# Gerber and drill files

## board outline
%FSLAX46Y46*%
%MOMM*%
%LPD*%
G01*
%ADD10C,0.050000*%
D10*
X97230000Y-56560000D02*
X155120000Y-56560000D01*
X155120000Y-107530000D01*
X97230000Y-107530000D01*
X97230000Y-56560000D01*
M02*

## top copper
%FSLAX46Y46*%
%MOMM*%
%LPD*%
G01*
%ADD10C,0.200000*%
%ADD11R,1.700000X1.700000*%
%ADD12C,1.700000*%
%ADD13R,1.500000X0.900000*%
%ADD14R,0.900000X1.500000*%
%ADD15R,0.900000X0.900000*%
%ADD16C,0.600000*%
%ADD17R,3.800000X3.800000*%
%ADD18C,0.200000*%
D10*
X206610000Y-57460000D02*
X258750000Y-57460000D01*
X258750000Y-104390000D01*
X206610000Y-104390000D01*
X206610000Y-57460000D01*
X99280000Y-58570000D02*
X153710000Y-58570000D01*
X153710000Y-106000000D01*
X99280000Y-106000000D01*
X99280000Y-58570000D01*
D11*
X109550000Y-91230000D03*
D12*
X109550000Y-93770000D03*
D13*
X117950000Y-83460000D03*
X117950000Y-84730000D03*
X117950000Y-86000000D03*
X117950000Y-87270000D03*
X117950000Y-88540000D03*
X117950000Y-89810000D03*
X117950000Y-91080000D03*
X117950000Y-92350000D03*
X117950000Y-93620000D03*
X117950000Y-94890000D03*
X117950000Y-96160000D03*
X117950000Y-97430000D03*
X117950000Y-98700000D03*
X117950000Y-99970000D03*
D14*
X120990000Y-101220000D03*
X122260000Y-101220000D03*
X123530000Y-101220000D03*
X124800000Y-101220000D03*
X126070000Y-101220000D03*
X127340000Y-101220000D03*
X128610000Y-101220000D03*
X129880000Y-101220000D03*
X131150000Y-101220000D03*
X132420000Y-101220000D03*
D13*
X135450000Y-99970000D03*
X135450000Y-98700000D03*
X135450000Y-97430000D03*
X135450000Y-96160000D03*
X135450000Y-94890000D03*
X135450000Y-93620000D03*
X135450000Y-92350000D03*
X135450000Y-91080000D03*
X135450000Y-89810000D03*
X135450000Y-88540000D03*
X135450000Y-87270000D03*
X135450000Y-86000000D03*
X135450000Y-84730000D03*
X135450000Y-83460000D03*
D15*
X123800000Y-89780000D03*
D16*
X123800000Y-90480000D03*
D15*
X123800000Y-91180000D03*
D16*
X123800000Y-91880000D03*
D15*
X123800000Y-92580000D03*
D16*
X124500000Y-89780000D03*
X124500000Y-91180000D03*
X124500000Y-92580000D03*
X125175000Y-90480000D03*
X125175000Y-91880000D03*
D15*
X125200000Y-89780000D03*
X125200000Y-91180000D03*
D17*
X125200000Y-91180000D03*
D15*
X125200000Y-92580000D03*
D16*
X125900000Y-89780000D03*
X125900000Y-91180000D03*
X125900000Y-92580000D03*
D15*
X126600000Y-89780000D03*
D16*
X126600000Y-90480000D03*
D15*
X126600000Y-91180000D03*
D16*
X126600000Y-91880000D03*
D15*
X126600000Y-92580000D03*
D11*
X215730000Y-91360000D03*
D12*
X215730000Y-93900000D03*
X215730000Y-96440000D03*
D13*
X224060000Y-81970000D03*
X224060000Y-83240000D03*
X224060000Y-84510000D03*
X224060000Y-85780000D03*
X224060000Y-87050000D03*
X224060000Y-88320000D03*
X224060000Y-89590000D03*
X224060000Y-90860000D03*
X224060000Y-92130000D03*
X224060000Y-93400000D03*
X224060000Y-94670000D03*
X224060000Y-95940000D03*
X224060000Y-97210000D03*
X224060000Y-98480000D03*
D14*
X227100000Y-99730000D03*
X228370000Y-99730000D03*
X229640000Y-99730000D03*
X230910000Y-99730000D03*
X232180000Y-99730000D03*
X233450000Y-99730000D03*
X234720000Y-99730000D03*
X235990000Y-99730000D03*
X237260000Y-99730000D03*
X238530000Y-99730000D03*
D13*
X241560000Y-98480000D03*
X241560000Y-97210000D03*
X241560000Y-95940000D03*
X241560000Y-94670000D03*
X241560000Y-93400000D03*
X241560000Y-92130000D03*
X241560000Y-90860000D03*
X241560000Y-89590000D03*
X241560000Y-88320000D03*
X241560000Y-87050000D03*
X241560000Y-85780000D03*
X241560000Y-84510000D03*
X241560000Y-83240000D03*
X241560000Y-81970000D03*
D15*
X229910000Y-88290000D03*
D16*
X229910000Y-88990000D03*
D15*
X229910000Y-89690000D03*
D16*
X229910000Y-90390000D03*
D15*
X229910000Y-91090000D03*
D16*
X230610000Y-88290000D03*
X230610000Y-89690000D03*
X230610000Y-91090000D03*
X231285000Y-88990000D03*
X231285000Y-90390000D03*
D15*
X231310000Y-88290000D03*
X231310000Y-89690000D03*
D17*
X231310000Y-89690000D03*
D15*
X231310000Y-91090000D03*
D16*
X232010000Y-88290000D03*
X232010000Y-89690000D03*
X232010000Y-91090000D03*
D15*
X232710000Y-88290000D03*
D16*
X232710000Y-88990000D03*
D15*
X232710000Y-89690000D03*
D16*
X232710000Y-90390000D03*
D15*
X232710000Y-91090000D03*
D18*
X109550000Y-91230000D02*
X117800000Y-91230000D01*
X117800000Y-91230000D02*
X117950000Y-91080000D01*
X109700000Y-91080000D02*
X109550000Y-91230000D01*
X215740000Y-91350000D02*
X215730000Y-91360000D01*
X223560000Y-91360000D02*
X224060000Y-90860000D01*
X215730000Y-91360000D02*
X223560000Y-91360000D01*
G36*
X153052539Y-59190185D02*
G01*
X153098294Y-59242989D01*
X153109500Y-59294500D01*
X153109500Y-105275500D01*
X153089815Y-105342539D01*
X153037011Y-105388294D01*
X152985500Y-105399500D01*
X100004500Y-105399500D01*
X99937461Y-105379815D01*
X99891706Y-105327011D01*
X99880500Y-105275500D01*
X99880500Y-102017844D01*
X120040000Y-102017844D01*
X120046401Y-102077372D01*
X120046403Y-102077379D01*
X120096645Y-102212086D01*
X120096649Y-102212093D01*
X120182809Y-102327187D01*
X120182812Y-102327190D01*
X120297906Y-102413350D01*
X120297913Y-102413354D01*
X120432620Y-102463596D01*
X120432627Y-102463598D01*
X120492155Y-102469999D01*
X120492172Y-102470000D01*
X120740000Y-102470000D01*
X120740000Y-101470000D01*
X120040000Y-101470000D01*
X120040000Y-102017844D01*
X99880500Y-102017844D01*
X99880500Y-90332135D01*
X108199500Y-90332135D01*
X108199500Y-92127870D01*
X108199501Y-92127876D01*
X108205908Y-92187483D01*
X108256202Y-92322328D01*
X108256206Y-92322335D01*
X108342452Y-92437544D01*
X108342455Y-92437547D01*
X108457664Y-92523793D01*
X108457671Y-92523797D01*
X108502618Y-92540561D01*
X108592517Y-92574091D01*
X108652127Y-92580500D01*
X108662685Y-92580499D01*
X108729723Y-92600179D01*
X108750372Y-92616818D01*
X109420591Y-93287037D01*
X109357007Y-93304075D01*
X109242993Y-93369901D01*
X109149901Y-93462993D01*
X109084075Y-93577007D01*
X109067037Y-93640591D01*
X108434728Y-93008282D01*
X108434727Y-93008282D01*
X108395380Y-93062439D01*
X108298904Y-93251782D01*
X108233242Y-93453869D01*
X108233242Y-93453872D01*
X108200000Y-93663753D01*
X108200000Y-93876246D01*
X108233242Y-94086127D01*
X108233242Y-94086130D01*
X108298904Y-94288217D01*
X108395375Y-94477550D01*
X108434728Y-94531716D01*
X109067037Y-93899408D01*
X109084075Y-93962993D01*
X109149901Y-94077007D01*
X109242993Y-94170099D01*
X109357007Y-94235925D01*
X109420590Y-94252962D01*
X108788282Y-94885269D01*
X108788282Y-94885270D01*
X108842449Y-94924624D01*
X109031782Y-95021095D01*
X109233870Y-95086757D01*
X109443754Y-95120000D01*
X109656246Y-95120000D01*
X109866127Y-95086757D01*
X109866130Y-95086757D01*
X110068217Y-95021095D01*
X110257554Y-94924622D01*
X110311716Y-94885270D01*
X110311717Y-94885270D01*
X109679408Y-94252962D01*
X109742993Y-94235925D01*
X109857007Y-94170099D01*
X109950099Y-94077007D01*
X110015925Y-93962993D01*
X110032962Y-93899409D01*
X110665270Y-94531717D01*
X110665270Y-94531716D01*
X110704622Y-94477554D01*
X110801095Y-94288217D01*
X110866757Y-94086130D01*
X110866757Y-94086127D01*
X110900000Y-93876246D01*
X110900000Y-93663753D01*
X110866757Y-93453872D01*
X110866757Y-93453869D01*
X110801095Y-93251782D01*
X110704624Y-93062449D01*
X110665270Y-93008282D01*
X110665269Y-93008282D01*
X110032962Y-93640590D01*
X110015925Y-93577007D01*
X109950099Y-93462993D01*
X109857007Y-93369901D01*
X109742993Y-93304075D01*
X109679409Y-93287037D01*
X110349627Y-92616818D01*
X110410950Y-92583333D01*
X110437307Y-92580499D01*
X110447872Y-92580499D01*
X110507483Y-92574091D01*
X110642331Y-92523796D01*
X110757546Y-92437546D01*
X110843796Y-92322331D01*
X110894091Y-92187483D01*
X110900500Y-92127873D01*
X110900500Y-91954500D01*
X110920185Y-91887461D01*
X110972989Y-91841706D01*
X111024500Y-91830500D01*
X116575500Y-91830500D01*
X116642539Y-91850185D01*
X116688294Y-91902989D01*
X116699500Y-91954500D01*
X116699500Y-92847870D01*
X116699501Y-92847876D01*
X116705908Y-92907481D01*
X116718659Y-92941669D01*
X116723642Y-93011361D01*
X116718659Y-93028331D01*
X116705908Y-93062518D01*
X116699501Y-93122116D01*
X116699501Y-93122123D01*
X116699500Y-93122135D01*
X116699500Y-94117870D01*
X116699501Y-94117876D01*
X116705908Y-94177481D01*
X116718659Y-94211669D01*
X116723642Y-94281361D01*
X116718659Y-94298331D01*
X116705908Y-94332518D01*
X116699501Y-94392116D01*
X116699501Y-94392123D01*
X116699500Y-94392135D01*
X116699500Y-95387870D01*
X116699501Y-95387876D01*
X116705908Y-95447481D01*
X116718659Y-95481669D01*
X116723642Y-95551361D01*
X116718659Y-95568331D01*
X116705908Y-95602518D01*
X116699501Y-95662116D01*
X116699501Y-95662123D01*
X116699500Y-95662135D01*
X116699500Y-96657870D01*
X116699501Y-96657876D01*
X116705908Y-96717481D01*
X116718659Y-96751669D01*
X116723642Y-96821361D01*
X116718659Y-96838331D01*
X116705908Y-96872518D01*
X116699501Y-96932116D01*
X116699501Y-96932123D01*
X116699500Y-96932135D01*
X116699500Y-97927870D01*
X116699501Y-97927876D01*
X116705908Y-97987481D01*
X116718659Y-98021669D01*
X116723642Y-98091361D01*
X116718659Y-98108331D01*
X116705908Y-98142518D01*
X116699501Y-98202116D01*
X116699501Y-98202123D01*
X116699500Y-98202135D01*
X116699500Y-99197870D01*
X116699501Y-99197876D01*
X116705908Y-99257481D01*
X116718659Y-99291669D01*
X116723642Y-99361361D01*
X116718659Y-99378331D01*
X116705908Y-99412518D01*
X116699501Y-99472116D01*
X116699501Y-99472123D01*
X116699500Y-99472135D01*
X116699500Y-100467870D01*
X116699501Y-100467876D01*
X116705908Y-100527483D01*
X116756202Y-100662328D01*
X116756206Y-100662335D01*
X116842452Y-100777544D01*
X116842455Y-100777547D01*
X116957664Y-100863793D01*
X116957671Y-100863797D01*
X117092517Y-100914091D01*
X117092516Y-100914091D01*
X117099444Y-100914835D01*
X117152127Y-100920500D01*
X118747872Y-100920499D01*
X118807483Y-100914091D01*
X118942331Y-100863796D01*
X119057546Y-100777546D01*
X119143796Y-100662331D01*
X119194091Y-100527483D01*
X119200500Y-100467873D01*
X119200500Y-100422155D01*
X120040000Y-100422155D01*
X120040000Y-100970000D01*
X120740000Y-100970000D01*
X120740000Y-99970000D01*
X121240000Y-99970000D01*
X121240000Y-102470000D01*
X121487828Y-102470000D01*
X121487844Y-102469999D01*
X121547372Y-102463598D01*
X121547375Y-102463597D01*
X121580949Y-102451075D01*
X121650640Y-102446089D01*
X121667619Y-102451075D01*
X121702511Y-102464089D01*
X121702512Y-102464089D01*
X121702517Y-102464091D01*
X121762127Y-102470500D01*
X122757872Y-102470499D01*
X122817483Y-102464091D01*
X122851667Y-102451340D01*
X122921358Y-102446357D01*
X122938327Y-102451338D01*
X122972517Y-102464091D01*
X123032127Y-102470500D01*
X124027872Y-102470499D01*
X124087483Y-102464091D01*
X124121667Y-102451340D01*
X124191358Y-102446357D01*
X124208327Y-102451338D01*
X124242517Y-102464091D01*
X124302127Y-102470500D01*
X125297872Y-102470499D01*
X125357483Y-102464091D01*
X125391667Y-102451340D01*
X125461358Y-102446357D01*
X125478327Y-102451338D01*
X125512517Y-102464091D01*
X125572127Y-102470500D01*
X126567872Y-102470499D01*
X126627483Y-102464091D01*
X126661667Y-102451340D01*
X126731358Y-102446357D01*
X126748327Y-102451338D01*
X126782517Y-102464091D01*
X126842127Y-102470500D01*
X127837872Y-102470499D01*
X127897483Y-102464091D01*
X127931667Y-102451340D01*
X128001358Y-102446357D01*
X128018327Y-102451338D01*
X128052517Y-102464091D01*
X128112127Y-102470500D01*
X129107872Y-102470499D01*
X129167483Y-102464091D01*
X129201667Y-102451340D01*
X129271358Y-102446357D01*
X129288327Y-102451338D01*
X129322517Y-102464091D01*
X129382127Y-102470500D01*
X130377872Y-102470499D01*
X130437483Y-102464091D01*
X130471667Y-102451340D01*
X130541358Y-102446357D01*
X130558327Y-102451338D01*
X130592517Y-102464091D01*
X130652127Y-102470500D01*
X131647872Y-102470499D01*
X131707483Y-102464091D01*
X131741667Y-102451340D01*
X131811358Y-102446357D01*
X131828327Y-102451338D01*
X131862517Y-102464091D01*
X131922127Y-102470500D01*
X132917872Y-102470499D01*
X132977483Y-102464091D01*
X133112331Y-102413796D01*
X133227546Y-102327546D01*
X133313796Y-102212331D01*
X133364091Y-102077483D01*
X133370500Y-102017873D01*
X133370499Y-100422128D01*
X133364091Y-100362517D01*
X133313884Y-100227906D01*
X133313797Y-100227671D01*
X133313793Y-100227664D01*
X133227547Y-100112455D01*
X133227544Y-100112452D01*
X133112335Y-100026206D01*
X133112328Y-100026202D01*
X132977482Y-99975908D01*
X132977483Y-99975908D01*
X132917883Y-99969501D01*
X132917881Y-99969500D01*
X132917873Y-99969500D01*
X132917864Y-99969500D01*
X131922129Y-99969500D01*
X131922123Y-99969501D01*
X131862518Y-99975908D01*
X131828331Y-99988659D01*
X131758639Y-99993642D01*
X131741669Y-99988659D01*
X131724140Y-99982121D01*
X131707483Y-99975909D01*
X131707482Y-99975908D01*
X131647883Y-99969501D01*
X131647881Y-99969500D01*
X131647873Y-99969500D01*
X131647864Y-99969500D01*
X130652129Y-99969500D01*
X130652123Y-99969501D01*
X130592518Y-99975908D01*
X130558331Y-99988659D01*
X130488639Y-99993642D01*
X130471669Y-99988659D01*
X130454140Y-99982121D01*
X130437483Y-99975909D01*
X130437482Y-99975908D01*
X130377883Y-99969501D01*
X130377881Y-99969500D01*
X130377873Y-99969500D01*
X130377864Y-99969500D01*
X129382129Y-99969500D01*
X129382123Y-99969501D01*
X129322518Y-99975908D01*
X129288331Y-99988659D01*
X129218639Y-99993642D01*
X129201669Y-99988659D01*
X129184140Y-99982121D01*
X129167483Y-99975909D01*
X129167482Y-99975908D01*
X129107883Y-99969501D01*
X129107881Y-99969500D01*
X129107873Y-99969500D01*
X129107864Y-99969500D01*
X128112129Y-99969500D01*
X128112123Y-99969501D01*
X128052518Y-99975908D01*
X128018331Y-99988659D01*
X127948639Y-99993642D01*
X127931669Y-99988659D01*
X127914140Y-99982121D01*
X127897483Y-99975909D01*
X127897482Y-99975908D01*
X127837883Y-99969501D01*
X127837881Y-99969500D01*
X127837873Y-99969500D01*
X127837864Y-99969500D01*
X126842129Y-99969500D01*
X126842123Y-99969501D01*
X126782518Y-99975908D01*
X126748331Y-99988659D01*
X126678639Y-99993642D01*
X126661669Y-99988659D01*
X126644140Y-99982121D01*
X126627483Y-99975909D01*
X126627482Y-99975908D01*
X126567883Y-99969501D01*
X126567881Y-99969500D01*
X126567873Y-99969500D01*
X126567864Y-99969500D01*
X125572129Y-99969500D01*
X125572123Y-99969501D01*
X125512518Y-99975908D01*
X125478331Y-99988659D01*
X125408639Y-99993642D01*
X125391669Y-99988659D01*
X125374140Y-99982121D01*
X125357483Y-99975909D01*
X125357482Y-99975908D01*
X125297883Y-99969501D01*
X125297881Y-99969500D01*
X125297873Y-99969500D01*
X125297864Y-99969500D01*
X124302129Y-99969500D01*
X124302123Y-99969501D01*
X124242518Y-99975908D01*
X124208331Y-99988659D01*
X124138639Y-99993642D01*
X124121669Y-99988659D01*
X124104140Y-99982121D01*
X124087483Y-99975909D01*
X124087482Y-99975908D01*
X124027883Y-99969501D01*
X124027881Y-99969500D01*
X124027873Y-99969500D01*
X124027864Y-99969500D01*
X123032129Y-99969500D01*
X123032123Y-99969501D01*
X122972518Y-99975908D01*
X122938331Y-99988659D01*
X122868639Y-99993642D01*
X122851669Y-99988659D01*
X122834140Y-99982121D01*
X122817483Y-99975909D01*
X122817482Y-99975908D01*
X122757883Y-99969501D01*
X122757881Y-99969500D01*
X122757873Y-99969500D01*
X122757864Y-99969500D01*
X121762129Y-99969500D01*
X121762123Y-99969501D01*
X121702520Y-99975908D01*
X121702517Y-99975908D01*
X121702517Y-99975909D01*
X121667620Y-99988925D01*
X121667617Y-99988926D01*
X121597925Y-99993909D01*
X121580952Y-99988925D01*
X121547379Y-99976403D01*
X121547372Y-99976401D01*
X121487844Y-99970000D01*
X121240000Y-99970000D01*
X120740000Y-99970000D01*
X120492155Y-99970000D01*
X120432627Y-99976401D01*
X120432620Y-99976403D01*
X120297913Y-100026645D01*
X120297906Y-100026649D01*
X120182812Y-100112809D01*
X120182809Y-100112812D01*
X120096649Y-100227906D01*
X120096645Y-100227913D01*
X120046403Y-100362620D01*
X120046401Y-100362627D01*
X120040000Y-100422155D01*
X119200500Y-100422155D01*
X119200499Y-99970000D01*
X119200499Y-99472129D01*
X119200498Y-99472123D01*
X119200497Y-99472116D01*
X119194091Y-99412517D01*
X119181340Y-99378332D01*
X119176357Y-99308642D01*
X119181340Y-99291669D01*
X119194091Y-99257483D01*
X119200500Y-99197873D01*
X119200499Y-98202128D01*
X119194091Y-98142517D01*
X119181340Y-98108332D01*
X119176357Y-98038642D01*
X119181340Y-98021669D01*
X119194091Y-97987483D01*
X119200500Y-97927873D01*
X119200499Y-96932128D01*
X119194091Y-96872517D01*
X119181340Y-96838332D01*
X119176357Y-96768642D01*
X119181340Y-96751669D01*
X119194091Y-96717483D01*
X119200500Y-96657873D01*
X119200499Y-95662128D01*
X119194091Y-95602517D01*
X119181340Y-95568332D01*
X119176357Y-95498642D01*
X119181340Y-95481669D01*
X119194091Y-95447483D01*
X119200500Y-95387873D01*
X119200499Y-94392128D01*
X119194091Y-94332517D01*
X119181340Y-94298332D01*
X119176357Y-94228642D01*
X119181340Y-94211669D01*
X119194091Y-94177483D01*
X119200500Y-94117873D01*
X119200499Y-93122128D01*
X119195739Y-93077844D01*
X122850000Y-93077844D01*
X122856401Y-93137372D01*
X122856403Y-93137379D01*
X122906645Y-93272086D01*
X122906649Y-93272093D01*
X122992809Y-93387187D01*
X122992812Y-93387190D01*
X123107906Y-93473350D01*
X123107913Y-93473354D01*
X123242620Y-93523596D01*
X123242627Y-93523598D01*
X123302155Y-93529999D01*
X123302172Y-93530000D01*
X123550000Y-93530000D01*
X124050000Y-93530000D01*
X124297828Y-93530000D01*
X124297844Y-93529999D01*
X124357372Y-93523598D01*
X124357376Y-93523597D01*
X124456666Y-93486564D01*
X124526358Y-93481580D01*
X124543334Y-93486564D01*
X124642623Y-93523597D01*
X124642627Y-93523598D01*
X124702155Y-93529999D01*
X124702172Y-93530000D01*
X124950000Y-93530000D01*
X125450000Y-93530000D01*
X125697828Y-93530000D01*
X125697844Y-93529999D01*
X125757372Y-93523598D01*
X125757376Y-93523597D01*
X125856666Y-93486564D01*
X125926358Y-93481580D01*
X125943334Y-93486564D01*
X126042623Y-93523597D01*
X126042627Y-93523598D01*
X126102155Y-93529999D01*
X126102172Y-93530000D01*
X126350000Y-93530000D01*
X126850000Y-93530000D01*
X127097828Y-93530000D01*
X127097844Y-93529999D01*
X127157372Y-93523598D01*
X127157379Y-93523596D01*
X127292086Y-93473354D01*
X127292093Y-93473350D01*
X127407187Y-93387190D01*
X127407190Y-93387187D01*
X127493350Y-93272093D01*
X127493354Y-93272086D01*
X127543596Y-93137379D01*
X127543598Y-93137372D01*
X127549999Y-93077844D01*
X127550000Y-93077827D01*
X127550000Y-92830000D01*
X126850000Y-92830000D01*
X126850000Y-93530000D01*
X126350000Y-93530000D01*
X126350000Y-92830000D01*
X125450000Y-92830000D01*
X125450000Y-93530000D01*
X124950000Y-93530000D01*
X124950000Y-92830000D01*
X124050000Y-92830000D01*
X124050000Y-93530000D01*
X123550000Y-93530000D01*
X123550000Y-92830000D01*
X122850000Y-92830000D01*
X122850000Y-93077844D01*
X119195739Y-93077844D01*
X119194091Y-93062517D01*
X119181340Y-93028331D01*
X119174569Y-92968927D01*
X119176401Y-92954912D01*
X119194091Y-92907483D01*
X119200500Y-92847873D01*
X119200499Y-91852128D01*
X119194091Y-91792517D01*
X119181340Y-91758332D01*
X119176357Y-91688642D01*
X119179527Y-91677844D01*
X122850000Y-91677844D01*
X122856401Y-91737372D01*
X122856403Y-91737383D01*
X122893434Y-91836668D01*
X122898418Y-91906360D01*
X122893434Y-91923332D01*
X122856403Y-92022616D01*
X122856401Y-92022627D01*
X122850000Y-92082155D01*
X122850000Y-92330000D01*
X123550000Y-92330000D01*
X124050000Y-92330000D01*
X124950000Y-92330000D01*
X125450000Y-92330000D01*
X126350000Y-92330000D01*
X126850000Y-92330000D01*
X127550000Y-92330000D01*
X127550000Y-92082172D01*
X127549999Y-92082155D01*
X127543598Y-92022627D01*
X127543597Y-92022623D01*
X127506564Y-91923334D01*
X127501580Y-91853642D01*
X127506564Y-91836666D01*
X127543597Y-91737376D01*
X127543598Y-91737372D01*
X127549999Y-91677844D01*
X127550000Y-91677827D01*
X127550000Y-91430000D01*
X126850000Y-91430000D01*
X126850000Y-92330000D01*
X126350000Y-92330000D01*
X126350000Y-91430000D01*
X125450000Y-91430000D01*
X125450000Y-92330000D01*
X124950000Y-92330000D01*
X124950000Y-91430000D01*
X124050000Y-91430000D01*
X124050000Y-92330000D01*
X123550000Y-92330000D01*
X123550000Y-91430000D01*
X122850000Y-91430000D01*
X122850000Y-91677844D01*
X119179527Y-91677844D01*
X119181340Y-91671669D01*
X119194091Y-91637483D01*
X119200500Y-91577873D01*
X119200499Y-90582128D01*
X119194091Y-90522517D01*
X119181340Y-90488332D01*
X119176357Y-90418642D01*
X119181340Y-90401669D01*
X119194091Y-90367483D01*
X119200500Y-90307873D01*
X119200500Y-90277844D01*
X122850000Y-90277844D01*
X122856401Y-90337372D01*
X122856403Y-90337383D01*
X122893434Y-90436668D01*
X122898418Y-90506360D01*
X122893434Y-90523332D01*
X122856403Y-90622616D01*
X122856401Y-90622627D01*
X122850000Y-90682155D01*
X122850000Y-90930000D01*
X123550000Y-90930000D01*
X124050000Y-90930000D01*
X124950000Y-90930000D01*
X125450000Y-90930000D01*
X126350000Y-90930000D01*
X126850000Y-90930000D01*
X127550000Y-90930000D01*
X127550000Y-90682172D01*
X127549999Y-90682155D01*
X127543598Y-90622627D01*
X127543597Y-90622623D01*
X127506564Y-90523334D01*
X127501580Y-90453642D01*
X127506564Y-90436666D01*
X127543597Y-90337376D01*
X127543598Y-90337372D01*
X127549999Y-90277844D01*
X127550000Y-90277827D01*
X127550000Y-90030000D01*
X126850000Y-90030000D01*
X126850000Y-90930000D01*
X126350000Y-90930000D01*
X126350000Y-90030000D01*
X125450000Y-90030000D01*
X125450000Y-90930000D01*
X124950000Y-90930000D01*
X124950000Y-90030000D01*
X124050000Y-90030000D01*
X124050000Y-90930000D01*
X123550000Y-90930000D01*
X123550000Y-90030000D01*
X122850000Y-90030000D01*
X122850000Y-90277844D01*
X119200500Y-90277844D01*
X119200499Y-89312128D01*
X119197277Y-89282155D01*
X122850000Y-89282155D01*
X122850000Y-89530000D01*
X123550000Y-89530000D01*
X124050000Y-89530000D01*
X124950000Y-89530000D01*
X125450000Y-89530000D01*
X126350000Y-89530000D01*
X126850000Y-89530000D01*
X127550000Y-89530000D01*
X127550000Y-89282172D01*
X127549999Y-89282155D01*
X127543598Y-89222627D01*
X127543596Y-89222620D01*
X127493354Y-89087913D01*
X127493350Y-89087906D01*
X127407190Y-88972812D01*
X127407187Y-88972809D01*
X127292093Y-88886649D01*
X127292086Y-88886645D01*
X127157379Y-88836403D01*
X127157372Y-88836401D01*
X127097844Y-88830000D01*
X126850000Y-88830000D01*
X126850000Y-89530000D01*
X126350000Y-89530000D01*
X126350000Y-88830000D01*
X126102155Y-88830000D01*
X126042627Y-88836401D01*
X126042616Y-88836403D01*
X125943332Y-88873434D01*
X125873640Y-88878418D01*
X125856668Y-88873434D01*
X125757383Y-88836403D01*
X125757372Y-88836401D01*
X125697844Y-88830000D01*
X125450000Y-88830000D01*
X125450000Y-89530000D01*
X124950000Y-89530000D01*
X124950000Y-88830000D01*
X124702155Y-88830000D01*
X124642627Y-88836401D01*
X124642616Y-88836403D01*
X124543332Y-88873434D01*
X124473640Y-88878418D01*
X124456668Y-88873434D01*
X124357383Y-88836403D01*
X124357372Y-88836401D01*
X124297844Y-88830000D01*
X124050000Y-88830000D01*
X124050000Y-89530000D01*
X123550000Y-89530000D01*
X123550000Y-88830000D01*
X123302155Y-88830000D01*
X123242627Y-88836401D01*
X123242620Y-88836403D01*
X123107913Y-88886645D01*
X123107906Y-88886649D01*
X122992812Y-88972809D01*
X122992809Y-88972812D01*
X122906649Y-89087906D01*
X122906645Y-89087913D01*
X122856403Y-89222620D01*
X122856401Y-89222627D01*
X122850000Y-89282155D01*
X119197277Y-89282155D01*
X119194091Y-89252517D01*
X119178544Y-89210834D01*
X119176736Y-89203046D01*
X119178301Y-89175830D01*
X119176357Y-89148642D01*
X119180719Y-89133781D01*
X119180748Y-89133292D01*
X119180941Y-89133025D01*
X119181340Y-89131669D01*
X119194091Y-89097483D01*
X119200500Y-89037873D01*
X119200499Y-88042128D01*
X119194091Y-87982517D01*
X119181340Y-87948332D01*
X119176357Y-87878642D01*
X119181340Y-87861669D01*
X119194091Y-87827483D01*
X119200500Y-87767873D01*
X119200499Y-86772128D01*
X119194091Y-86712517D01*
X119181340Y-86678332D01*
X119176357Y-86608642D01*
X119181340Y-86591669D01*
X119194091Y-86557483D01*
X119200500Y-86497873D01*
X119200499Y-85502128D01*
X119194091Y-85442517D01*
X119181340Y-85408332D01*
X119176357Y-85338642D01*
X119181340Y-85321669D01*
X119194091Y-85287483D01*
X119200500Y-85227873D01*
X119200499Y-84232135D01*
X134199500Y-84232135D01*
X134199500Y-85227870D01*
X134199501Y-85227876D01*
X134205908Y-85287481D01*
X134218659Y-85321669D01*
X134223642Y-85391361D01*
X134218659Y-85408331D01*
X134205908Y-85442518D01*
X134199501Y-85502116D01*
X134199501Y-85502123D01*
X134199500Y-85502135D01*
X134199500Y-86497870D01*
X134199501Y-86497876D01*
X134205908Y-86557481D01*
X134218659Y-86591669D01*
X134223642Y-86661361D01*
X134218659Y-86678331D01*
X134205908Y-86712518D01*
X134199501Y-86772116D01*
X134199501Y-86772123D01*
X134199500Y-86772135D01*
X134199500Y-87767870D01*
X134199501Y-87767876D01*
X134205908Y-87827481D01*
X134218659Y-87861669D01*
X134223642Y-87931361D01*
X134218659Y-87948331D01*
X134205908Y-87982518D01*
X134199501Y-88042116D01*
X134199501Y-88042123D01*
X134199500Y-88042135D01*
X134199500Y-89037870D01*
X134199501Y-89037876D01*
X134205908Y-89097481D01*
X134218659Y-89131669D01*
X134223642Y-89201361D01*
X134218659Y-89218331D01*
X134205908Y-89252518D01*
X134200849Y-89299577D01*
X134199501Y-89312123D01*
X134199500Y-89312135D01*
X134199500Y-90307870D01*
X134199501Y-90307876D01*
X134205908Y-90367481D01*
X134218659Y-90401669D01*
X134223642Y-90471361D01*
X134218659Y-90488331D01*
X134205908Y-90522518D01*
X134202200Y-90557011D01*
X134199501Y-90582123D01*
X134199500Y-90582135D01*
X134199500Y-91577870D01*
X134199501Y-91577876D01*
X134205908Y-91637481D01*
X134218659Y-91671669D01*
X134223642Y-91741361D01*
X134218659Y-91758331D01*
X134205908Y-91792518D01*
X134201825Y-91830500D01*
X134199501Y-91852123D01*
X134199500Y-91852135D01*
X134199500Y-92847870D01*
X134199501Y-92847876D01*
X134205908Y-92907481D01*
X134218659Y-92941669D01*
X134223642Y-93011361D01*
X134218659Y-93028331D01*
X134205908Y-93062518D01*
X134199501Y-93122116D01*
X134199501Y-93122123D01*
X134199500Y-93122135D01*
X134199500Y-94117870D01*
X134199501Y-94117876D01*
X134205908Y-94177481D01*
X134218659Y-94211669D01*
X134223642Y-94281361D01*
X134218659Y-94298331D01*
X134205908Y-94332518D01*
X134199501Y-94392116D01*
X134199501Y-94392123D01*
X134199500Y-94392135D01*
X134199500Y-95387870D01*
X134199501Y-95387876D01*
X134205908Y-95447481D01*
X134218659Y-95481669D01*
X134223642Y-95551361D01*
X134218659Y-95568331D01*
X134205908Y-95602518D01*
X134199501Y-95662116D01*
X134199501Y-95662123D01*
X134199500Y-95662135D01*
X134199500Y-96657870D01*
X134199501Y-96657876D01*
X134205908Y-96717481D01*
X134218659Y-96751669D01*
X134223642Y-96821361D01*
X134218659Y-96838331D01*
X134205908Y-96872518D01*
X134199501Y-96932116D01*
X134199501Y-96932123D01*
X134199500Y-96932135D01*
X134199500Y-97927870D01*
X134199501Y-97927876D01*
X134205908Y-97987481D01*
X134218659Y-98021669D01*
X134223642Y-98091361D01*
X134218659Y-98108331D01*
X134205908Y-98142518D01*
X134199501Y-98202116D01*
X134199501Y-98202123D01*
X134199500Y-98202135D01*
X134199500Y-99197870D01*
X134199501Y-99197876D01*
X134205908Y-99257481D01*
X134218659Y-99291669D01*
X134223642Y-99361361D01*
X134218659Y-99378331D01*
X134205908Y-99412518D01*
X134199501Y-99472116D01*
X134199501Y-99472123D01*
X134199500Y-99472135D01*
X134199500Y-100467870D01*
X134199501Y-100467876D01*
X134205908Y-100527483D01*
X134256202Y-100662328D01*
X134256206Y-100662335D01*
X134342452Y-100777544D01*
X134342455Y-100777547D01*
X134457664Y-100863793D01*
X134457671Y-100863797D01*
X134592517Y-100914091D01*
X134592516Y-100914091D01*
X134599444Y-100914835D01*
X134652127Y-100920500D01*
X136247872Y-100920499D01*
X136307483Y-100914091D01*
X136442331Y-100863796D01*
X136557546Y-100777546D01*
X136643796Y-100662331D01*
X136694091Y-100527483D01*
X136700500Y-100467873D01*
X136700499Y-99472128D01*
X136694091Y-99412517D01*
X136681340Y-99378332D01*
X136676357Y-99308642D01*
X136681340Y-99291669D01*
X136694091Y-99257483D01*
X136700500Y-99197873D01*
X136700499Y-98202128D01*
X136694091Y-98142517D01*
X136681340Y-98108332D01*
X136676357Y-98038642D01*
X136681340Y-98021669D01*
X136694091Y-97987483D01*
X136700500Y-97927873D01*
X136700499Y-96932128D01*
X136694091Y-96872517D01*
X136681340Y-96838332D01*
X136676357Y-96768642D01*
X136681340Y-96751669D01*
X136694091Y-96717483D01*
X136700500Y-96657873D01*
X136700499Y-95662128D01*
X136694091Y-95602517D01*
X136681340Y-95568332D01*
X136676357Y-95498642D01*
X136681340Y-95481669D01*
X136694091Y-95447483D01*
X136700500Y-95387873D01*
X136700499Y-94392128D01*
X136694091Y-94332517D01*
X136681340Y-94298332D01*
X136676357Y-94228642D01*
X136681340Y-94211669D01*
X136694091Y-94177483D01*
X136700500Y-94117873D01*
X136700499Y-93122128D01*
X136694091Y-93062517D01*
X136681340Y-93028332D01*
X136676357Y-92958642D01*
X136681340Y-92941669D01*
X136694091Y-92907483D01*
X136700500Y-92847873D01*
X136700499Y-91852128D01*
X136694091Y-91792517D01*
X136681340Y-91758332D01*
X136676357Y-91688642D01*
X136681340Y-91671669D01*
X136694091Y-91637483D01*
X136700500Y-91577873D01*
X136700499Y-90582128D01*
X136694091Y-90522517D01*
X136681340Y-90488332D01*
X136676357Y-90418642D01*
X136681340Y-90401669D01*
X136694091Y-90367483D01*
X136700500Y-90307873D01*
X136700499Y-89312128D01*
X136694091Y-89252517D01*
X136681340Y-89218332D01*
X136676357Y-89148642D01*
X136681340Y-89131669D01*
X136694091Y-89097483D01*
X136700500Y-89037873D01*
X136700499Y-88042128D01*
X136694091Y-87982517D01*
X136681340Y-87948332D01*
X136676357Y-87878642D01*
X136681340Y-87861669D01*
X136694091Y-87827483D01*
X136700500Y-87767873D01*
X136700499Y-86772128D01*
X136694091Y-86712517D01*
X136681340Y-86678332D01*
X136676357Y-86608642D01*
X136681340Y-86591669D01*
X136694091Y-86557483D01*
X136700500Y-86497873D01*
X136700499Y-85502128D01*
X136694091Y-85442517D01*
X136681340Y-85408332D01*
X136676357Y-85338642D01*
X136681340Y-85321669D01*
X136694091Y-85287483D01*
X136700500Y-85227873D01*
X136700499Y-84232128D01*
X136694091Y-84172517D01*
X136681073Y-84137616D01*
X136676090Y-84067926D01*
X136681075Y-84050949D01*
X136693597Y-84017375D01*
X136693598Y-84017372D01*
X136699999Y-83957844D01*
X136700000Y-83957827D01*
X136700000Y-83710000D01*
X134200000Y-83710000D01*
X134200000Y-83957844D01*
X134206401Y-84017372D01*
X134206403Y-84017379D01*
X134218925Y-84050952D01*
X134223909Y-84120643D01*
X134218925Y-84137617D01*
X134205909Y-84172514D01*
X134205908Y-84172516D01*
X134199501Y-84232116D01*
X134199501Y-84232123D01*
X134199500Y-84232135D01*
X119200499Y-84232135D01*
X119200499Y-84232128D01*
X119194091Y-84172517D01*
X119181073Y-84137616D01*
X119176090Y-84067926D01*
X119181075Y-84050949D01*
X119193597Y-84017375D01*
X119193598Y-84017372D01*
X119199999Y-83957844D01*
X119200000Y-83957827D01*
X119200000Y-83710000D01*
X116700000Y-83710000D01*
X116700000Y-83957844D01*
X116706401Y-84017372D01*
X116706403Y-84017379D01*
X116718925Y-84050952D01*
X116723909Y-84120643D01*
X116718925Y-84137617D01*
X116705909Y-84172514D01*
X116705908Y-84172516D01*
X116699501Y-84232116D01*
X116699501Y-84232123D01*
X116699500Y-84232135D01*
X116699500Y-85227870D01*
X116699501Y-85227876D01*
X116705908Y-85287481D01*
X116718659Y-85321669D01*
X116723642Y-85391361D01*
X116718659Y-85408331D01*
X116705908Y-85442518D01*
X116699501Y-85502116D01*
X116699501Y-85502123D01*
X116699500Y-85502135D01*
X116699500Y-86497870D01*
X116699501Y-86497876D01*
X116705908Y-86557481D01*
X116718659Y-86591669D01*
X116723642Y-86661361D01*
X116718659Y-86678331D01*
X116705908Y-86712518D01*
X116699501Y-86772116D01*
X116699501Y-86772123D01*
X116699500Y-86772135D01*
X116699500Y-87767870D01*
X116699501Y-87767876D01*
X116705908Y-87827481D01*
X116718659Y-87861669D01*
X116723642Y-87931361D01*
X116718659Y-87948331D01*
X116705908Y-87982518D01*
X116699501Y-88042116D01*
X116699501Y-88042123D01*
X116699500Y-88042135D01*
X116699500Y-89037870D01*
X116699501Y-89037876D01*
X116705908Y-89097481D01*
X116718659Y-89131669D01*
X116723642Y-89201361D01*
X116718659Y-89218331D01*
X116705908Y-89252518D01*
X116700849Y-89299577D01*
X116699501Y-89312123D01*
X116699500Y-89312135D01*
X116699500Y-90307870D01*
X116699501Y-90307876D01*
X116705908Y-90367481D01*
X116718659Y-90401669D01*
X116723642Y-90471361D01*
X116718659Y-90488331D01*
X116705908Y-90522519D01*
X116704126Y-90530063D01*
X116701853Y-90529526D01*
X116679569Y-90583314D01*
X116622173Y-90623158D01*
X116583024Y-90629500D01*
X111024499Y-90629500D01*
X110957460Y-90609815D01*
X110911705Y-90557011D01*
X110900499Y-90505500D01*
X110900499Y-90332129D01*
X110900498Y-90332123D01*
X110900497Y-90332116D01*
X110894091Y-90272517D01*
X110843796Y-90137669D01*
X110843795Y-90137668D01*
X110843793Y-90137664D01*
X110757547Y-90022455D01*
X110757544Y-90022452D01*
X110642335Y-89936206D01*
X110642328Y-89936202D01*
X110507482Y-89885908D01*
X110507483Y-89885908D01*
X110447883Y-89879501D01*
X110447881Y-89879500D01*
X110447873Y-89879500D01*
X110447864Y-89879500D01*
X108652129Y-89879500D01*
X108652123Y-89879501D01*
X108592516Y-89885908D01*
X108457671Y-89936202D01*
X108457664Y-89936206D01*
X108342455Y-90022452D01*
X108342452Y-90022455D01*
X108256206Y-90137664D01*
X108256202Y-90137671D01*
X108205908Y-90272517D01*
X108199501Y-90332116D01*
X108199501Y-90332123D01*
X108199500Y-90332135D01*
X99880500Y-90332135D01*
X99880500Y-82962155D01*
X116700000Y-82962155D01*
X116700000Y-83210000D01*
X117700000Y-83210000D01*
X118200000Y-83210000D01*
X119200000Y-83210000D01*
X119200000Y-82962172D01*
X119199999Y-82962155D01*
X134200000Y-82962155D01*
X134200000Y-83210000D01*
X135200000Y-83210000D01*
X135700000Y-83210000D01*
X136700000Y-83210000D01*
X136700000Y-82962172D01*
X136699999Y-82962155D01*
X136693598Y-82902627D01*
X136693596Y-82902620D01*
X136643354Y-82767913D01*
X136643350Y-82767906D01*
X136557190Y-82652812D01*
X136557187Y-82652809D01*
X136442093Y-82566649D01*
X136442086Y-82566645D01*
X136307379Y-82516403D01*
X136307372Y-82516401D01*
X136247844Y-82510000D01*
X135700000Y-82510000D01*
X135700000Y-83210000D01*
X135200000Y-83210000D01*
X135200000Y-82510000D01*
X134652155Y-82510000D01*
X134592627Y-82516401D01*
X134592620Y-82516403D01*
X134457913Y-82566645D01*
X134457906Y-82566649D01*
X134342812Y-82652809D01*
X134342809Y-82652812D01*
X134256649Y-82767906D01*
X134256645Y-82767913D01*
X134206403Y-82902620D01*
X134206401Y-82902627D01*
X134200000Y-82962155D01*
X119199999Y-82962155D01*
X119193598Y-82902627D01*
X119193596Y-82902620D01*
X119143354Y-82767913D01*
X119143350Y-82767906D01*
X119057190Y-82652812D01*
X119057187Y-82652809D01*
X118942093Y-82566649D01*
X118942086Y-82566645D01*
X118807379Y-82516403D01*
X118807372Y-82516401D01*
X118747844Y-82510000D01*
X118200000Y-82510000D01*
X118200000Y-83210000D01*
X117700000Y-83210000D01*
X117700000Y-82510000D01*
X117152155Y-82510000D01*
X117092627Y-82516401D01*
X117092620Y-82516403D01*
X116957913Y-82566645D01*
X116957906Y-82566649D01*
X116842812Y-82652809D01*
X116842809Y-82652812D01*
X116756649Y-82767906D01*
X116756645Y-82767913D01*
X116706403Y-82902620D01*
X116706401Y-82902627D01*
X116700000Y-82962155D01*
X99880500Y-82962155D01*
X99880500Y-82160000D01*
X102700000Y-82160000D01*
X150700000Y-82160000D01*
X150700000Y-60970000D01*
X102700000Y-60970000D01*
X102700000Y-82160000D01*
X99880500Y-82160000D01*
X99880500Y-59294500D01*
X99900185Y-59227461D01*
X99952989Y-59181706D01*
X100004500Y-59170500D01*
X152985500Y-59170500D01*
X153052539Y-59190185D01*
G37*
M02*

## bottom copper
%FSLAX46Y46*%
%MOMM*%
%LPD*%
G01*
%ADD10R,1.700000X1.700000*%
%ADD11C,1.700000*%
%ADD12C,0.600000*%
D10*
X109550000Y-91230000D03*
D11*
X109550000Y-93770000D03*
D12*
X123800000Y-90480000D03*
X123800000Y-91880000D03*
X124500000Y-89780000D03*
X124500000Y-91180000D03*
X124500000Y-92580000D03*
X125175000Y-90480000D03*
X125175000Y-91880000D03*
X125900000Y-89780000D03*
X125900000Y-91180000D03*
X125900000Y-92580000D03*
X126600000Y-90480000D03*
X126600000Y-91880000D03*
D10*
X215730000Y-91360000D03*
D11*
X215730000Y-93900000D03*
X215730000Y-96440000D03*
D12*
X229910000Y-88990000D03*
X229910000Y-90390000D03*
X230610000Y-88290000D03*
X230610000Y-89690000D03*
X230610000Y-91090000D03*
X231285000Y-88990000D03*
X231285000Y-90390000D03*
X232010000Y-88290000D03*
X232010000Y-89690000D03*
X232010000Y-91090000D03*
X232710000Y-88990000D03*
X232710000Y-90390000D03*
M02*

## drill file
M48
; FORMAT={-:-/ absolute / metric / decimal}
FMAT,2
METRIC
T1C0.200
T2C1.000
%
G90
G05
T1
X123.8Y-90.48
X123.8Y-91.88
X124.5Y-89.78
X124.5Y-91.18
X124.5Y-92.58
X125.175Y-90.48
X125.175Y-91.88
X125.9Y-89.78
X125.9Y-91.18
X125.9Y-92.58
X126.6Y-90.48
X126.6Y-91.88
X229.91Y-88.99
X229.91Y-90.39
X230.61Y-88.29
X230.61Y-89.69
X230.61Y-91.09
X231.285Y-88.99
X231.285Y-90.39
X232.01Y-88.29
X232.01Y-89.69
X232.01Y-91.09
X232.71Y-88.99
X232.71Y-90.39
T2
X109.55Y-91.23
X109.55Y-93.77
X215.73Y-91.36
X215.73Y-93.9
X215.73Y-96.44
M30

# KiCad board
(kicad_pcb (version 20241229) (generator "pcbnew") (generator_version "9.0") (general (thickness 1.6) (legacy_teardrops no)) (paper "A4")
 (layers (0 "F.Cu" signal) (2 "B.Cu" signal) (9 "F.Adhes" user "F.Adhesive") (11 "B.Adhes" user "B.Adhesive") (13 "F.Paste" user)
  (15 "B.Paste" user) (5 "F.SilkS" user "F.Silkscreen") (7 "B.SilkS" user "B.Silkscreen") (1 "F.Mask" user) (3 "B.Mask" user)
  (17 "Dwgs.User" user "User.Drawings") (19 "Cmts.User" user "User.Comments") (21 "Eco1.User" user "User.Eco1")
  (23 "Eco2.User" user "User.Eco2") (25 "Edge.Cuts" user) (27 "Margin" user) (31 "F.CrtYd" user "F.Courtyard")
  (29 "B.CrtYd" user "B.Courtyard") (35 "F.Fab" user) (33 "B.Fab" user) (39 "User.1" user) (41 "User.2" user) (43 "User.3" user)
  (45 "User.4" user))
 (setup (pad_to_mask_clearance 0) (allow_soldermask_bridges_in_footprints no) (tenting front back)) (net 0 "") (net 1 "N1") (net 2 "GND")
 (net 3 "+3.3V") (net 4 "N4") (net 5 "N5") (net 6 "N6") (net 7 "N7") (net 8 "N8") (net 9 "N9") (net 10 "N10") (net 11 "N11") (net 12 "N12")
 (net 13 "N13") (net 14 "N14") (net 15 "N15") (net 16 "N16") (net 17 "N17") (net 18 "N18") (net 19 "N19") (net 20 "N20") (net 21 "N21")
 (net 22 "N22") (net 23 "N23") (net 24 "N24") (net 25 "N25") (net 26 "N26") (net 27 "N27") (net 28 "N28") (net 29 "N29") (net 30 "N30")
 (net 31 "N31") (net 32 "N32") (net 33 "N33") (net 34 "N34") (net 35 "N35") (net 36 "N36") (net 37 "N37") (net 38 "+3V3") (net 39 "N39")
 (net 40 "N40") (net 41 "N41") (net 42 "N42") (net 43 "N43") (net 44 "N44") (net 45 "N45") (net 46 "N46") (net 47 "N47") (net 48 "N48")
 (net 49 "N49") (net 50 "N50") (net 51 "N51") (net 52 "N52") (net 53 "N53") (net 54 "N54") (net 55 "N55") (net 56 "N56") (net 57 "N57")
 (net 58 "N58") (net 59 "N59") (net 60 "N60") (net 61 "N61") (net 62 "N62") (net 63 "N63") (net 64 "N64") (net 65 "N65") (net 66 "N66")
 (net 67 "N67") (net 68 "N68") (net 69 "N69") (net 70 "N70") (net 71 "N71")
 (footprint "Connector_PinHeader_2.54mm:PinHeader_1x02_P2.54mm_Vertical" (layer "F.Cu") (at 109.55 91.23)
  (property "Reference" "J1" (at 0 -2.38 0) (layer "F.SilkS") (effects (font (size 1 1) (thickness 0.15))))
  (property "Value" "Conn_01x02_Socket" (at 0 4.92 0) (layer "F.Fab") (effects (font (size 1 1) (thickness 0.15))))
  (pad "1" thru_hole rect (at 0 0) (size 1.7 1.7) (drill 1) (layers "*.Cu" "*.Mask") (remove_unused_layers no) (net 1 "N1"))
  (pad "2" thru_hole circle (at 0 2.54) (size 1.7 1.7) (drill 1) (layers "*.Cu" "*.Mask") (remove_unused_layers no) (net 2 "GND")))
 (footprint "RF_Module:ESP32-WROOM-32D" (layer "F.Cu") (at 126.7 91.71)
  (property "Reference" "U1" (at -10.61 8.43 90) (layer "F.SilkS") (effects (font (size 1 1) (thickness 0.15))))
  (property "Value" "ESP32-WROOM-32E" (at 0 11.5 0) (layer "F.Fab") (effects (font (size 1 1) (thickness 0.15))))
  (pad "1" smd rect (at -8.75 -8.25) (size 1.5 0.9) (layers "F.Cu" "F.Mask" "F.Paste") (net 2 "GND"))
  (pad "2" smd rect (at -8.75 -6.98) (size 1.5 0.9) (layers "F.Cu" "F.Mask" "F.Paste") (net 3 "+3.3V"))
  (pad "3" smd rect (at -8.75 -5.71) (size 1.5 0.9) (layers "F.Cu" "F.Mask" "F.Paste") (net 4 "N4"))
  (pad "4" smd rect (at -8.75 -4.44) (size 1.5 0.9) (layers "F.Cu" "F.Mask" "F.Paste") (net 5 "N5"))
  (pad "5" smd rect (at -8.75 -3.17) (size 1.5 0.9) (layers "F.Cu" "F.Mask" "F.Paste") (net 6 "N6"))
  (pad "6" smd rect (at -8.75 -1.9) (size 1.5 0.9) (layers "F.Cu" "F.Mask" "F.Paste") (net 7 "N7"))
  (pad "7" smd rect (at -8.75 -0.63) (size 1.5 0.9) (layers "F.Cu" "F.Mask" "F.Paste") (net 1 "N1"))
  (pad "8" smd rect (at -8.75 0.64) (size 1.5 0.9) (layers "F.Cu" "F.Mask" "F.Paste") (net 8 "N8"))
  (pad "9" smd rect (at -8.75 1.91) (size 1.5 0.9) (layers "F.Cu" "F.Mask" "F.Paste") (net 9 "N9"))
  (pad "10" smd rect (at -8.75 3.18) (size 1.5 0.9) (layers "F.Cu" "F.Mask" "F.Paste") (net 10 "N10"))
  (pad "11" smd rect (at -8.75 4.45) (size 1.5 0.9) (layers "F.Cu" "F.Mask" "F.Paste") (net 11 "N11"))
  (pad "12" smd rect (at -8.75 5.72) (size 1.5 0.9) (layers "F.Cu" "F.Mask" "F.Paste") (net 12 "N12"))
  (pad "13" smd rect (at -8.75 6.99) (size 1.5 0.9) (layers "F.Cu" "F.Mask" "F.Paste") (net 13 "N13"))
  (pad "14" smd rect (at -8.75 8.26) (size 1.5 0.9) (layers "F.Cu" "F.Mask" "F.Paste") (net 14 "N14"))
  (pad "15" smd rect (at -5.71 9.51 90) (size 1.5 0.9) (layers "F.Cu" "F.Mask" "F.Paste") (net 2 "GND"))
  (pad "16" smd rect (at -4.44 9.51 90) (size 1.5 0.9) (layers "F.Cu" "F.Mask" "F.Paste") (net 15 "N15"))
  (pad "17" smd rect (at -3.17 9.51 90) (size 1.5 0.9) (layers "F.Cu" "F.Mask" "F.Paste") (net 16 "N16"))
  (pad "18" smd rect (at -1.9 9.51 90) (size 1.5 0.9) (layers "F.Cu" "F.Mask" "F.Paste") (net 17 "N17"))
  (pad "19" smd rect (at -0.63 9.51 90) (size 1.5 0.9) (layers "F.Cu" "F.Mask" "F.Paste") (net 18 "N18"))
  (pad "20" smd rect (at 0.64 9.51 90) (size 1.5 0.9) (layers "F.Cu" "F.Mask" "F.Paste") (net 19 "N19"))
  (pad "21" smd rect (at 1.91 9.51 90) (size 1.5 0.9) (layers "F.Cu" "F.Mask" "F.Paste") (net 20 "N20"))
  (pad "22" smd rect (at 3.18 9.51 90) (size 1.5 0.9) (layers "F.Cu" "F.Mask" "F.Paste") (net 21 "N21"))
  (pad "23" smd rect (at 4.45 9.51 90) (size 1.5 0.9) (layers "F.Cu" "F.Mask" "F.Paste") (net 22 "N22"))
  (pad "24" smd rect (at 5.72 9.51 90) (size 1.5 0.9) (layers "F.Cu" "F.Mask" "F.Paste") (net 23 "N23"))
  (pad "25" smd rect (at 8.75 8.26) (size 1.5 0.9) (layers "F.Cu" "F.Mask" "F.Paste") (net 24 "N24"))
  (pad "26" smd rect (at 8.75 6.99) (size 1.5 0.9) (layers "F.Cu" "F.Mask" "F.Paste") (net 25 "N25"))
  (pad "27" smd rect (at 8.75 5.72) (size 1.5 0.9) (layers "F.Cu" "F.Mask" "F.Paste") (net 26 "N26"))
  (pad "28" smd rect (at 8.75 4.45) (size 1.5 0.9) (layers "F.Cu" "F.Mask" "F.Paste") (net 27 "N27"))
  (pad "29" smd rect (at 8.75 3.18) (size 1.5 0.9) (layers "F.Cu" "F.Mask" "F.Paste") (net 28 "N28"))
  (pad "30" smd rect (at 8.75 1.91) (size 1.5 0.9) (layers "F.Cu" "F.Mask" "F.Paste") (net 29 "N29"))
  (pad "31" smd rect (at 8.75 0.64) (size 1.5 0.9) (layers "F.Cu" "F.Mask" "F.Paste") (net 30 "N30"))
  (pad "32" smd rect (at 8.75 -0.63) (size 1.5 0.9) (layers "F.Cu" "F.Mask" "F.Paste") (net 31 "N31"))
  (pad "33" smd rect (at 8.75 -1.9) (size 1.5 0.9) (layers "F.Cu" "F.Mask" "F.Paste") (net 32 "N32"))
  (pad "34" smd rect (at 8.75 -3.17) (size 1.5 0.9) (layers "F.Cu" "F.Mask" "F.Paste") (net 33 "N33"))
  (pad "35" smd rect (at 8.75 -4.44) (size 1.5 0.9) (layers "F.Cu" "F.Mask" "F.Paste") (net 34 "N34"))
  (pad "36" smd rect (at 8.75 -5.71) (size 1.5 0.9) (layers "F.Cu" "F.Mask" "F.Paste") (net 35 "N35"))
  (pad "37" smd rect (at 8.75 -6.98) (size 1.5 0.9) (layers "F.Cu" "F.Mask" "F.Paste") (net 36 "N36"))
  (pad "38" smd rect (at 8.75 -8.25) (size 1.5 0.9) (layers "F.Cu" "F.Mask" "F.Paste") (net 2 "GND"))
  (pad "39" smd rect (at -2.9 -1.93) (size 0.9 0.9) (layers "F.Cu" "F.Paste") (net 2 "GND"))
  (pad "39" thru_hole circle (at -2.9 -1.23) (size 0.6 0.6) (drill 0.2) (layers "*.Cu" "F.Mask") (remove_unused_layers no) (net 2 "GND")
   (zone_connect 2))
  (pad "39" smd rect (at -2.9 -0.53) (size 0.9 0.9) (layers "F.Cu" "F.Paste") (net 2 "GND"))
  (pad "39" thru_hole circle (at -2.9 0.17) (size 0.6 0.6) (drill 0.2) (layers "*.Cu" "F.Mask") (remove_unused_layers no) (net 2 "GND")
   (zone_connect 2))
  (pad "39" smd rect (at -2.9 0.87) (size 0.9 0.9) (layers "F.Cu" "F.Paste") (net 2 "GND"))
  (pad "39" thru_hole circle (at -2.2 -1.93) (size 0.6 0.6) (drill 0.2) (layers "*.Cu" "F.Mask") (remove_unused_layers no) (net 2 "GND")
   (zone_connect 2))
  (pad "39" thru_hole circle (at -2.2 -0.53) (size 0.6 0.6) (drill 0.2) (layers "*.Cu" "F.Mask") (remove_unused_layers no) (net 2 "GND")
   (zone_connect 2))
  (pad "39" thru_hole circle (at -2.2 0.87) (size 0.6 0.6) (drill 0.2) (layers "*.Cu" "F.Mask") (remove_unused_layers no) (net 2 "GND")
   (zone_connect 2))
  (pad "39" thru_hole circle (at -1.525 -1.23) (size 0.6 0.6) (drill 0.2) (layers "*.Cu" "F.Mask") (remove_unused_layers no) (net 2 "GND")
   (zone_connect 2))
  (pad "39" thru_hole circle (at -1.525 0.17) (size 0.6 0.6) (drill 0.2) (layers "*.Cu" "F.Mask") (remove_unused_layers no) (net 2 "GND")
   (zone_connect 2))
  (pad "39" smd rect (at -1.5 -1.93) (size 0.9 0.9) (layers "F.Cu" "F.Paste") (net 2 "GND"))
  (pad "39" smd rect (at -1.5 -0.53) (size 0.9 0.9) (layers "F.Cu" "F.Paste") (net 2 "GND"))
  (pad "39" smd rect (at -1.5 -0.53) (size 3.8 3.8) (layers "F.Cu" "F.Mask") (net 2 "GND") (zone_connect 2))
  (pad "39" smd rect (at -1.5 0.87) (size 0.9 0.9) (layers "F.Cu" "F.Paste") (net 2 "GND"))
  (pad "39" thru_hole circle (at -0.8 -1.93) (size 0.6 0.6) (drill 0.2) (layers "*.Cu" "F.Mask") (remove_unused_layers no) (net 2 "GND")
   (zone_connect 2))
  (pad "39" thru_hole circle (at -0.8 -0.53) (size 0.6 0.6) (drill 0.2) (layers "*.Cu" "F.Mask") (remove_unused_layers no) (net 2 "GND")
   (zone_connect 2))
  (pad "39" thru_hole circle (at -0.8 0.87) (size 0.6 0.6) (drill 0.2) (layers "*.Cu" "F.Mask") (remove_unused_layers no) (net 2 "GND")
   (zone_connect 2))
  (pad "39" smd rect (at -0.1 -1.93) (size 0.9 0.9) (layers "F.Cu" "F.Paste") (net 2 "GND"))
  (pad "39" thru_hole circle (at -0.1 -1.23) (size 0.6 0.6) (drill 0.2) (layers "*.Cu" "F.Mask") (remove_unused_layers no) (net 2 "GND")
   (zone_connect 2))
  (pad "39" smd rect (at -0.1 -0.53) (size 0.9 0.9) (layers "F.Cu" "F.Paste") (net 2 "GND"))
  (pad "39" thru_hole circle (at -0.1 0.17) (size 0.6 0.6) (drill 0.2) (layers "*.Cu" "F.Mask") (remove_unused_layers no) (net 2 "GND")
   (zone_connect 2))
  (pad "39" smd rect (at -0.1 0.87) (size 0.9 0.9) (layers "F.Cu" "F.Paste") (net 2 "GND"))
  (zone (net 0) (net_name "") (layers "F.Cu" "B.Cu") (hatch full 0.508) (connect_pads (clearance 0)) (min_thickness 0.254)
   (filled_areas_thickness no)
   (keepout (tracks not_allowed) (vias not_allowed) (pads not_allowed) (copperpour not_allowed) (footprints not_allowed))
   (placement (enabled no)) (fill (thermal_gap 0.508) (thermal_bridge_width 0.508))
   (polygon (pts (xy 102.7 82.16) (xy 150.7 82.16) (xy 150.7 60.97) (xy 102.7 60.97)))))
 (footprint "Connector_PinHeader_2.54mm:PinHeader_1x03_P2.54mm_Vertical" (layer "F.Cu") (at 215.73 91.36)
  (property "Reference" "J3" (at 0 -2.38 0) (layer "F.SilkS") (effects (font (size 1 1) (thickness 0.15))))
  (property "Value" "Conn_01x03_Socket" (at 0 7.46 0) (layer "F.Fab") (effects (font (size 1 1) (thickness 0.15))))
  (pad "1" thru_hole rect (at 0 0) (size 1.7 1.7) (drill 1) (layers "*.Cu" "*.Mask") (remove_unused_layers no) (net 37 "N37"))
  (pad "2" thru_hole circle (at 0 2.54) (size 1.7 1.7) (drill 1) (layers "*.Cu" "*.Mask") (remove_unused_layers no) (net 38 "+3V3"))
  (pad "3" thru_hole circle (at 0 5.08) (size 1.7 1.7) (drill 1) (layers "*.Cu" "*.Mask") (remove_unused_layers no) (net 2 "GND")))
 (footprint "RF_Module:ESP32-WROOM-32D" (layer "F.Cu") (at 232.81 90.22)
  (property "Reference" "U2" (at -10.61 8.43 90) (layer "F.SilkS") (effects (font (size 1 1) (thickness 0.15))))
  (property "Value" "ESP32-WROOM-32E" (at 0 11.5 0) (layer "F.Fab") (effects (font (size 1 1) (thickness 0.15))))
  (pad "1" smd rect (at -8.75 -8.25) (size 1.5 0.9) (layers "F.Cu" "F.Mask" "F.Paste") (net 2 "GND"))
  (pad "2" smd rect (at -8.75 -6.98) (size 1.5 0.9) (layers "F.Cu" "F.Mask" "F.Paste") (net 3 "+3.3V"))
  (pad "3" smd rect (at -8.75 -5.71) (size 1.5 0.9) (layers "F.Cu" "F.Mask" "F.Paste") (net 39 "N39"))
  (pad "4" smd rect (at -8.75 -4.44) (size 1.5 0.9) (layers "F.Cu" "F.Mask" "F.Paste") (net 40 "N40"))
  (pad "5" smd rect (at -8.75 -3.17) (size 1.5 0.9) (layers "F.Cu" "F.Mask" "F.Paste") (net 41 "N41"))
  (pad "6" smd rect (at -8.75 -1.9) (size 1.5 0.9) (layers "F.Cu" "F.Mask" "F.Paste") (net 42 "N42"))
  (pad "7" smd rect (at -8.75 -0.63) (size 1.5 0.9) (layers "F.Cu" "F.Mask" "F.Paste") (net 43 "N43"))
  (pad "8" smd rect (at -8.75 0.64) (size 1.5 0.9) (layers "F.Cu" "F.Mask" "F.Paste") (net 37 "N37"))
  (pad "9" smd rect (at -8.75 1.91) (size 1.5 0.9) (layers "F.Cu" "F.Mask" "F.Paste") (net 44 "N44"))
  (pad "10" smd rect (at -8.75 3.18) (size 1.5 0.9) (layers "F.Cu" "F.Mask" "F.Paste") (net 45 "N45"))
  (pad "11" smd rect (at -8.75 4.45) (size 1.5 0.9) (layers "F.Cu" "F.Mask" "F.Paste") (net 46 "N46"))
  (pad "12" smd rect (at -8.75 5.72) (size 1.5 0.9) (layers "F.Cu" "F.Mask" "F.Paste") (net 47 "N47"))
  (pad "13" smd rect (at -8.75 6.99) (size 1.5 0.9) (layers "F.Cu" "F.Mask" "F.Paste") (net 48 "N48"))
  (pad "14" smd rect (at -8.75 8.26) (size 1.5 0.9) (layers "F.Cu" "F.Mask" "F.Paste") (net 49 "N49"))
  (pad "15" smd rect (at -5.71 9.51 90) (size 1.5 0.9) (layers "F.Cu" "F.Mask" "F.Paste") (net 2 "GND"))
  (pad "16" smd rect (at -4.44 9.51 90) (size 1.5 0.9) (layers "F.Cu" "F.Mask" "F.Paste") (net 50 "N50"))
  (pad "17" smd rect (at -3.17 9.51 90) (size 1.5 0.9) (layers "F.Cu" "F.Mask" "F.Paste") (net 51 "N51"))
  (pad "18" smd rect (at -1.9 9.51 90) (size 1.5 0.9) (layers "F.Cu" "F.Mask" "F.Paste") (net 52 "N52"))
  (pad "19" smd rect (at -0.63 9.51 90) (size 1.5 0.9) (layers "F.Cu" "F.Mask" "F.Paste") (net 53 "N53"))
  (pad "20" smd rect (at 0.64 9.51 90) (size 1.5 0.9) (layers "F.Cu" "F.Mask" "F.Paste") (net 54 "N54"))
  (pad "21" smd rect (at 1.91 9.51 90) (size 1.5 0.9) (layers "F.Cu" "F.Mask" "F.Paste") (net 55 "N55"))
  (pad "22" smd rect (at 3.18 9.51 90) (size 1.5 0.9) (layers "F.Cu" "F.Mask" "F.Paste") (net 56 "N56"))
  (pad "23" smd rect (at 4.45 9.51 90) (size 1.5 0.9) (layers "F.Cu" "F.Mask" "F.Paste") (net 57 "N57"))
  (pad "24" smd rect (at 5.72 9.51 90) (size 1.5 0.9) (layers "F.Cu" "F.Mask" "F.Paste") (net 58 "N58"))
  (pad "25" smd rect (at 8.75 8.26) (size 1.5 0.9) (layers "F.Cu" "F.Mask" "F.Paste") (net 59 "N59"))
  (pad "26" smd rect (at 8.75 6.99) (size 1.5 0.9) (layers "F.Cu" "F.Mask" "F.Paste") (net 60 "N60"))
  (pad "27" smd rect (at 8.75 5.72) (size 1.5 0.9) (layers "F.Cu" "F.Mask" "F.Paste") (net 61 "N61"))
  (pad "28" smd rect (at 8.75 4.45) (size 1.5 0.9) (layers "F.Cu" "F.Mask" "F.Paste") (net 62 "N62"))
  (pad "29" smd rect (at 8.75 3.18) (size 1.5 0.9) (layers "F.Cu" "F.Mask" "F.Paste") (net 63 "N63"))
  (pad "30" smd rect (at 8.75 1.91) (size 1.5 0.9) (layers "F.Cu" "F.Mask" "F.Paste") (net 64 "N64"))
  (pad "31" smd rect (at 8.75 0.64) (size 1.5 0.9) (layers "F.Cu" "F.Mask" "F.Paste") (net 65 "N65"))
  (pad "32" smd rect (at 8.75 -0.63) (size 1.5 0.9) (layers "F.Cu" "F.Mask" "F.Paste") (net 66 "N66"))
  (pad "33" smd rect (at 8.75 -1.9) (size 1.5 0.9) (layers "F.Cu" "F.Mask" "F.Paste") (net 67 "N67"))
  (pad "34" smd rect (at 8.75 -3.17) (size 1.5 0.9) (layers "F.Cu" "F.Mask" "F.Paste") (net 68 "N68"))
  (pad "35" smd rect (at 8.75 -4.44) (size 1.5 0.9) (layers "F.Cu" "F.Mask" "F.Paste") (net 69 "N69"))
  (pad "36" smd rect (at 8.75 -5.71) (size 1.5 0.9) (layers "F.Cu" "F.Mask" "F.Paste") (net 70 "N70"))
  (pad "37" smd rect (at 8.75 -6.98) (size 1.5 0.9) (layers "F.Cu" "F.Mask" "F.Paste") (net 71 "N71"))
  (pad "38" smd rect (at 8.75 -8.25) (size 1.5 0.9) (layers "F.Cu" "F.Mask" "F.Paste") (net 2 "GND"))
  (pad "39" smd rect (at -2.9 -1.93) (size 0.9 0.9) (layers "F.Cu" "F.Paste") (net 2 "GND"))
  (pad "39" thru_hole circle (at -2.9 -1.23) (size 0.6 0.6) (drill 0.2) (layers "*.Cu" "F.Mask") (remove_unused_layers no) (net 2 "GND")
   (zone_connect 2))
  (pad "39" smd rect (at -2.9 -0.53) (size 0.9 0.9) (layers "F.Cu" "F.Paste") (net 2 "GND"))
  (pad "39" thru_hole circle (at -2.9 0.17) (size 0.6 0.6) (drill 0.2) (layers "*.Cu" "F.Mask") (remove_unused_layers no) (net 2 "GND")
   (zone_connect 2))
  (pad "39" smd rect (at -2.9 0.87) (size 0.9 0.9) (layers "F.Cu" "F.Paste") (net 2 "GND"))
  (pad "39" thru_hole circle (at -2.2 -1.93) (size 0.6 0.6) (drill 0.2) (layers "*.Cu" "F.Mask") (remove_unused_layers no) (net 2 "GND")
   (zone_connect 2))
  (pad "39" thru_hole circle (at -2.2 -0.53) (size 0.6 0.6) (drill 0.2) (layers "*.Cu" "F.Mask") (remove_unused_layers no) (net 2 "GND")
   (zone_connect 2))
  (pad "39" thru_hole circle (at -2.2 0.87) (size 0.6 0.6) (drill 0.2) (layers "*.Cu" "F.Mask") (remove_unused_layers no) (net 2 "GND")
   (zone_connect 2))
  (pad "39" thru_hole circle (at -1.525 -1.23) (size 0.6 0.6) (drill 0.2) (layers "*.Cu" "F.Mask") (remove_unused_layers no) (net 2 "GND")
   (zone_connect 2))
  (pad "39" thru_hole circle (at -1.525 0.17) (size 0.6 0.6) (drill 0.2) (layers "*.Cu" "F.Mask") (remove_unused_layers no) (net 2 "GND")
   (zone_connect 2))
  (pad "39" smd rect (at -1.5 -1.93) (size 0.9 0.9) (layers "F.Cu" "F.Paste") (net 2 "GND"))
  (pad "39" smd rect (at -1.5 -0.53) (size 0.9 0.9) (layers "F.Cu" "F.Paste") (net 2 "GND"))
  (pad "39" smd rect (at -1.5 -0.53) (size 3.8 3.8) (layers "F.Cu" "F.Mask") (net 2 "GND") (zone_connect 2))
  (pad "39" smd rect (at -1.5 0.87) (size 0.9 0.9) (layers "F.Cu" "F.Paste") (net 2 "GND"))
  (pad "39" thru_hole circle (at -0.8 -1.93) (size 0.6 0.6) (drill 0.2) (layers "*.Cu" "F.Mask") (remove_unused_layers no) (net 2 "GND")
   (zone_connect 2))
  (pad "39" thru_hole circle (at -0.8 -0.53) (size 0.6 0.6) (drill 0.2) (layers "*.Cu" "F.Mask") (remove_unused_layers no) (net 2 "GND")
   (zone_connect 2))
  (pad "39" thru_hole circle (at -0.8 0.87) (size 0.6 0.6) (drill 0.2) (layers "*.Cu" "F.Mask") (remove_unused_layers no) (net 2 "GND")
   (zone_connect 2))
  (pad "39" smd rect (at -0.1 -1.93) (size 0.9 0.9) (layers "F.Cu" "F.Paste") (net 2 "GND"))
  (pad "39" thru_hole circle (at -0.1 -1.23) (size 0.6 0.6) (drill 0.2) (layers "*.Cu" "F.Mask") (remove_unused_layers no) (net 2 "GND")
   (zone_connect 2))
  (pad "39" smd rect (at -0.1 -0.53) (size 0.9 0.9) (layers "F.Cu" "F.Paste") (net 2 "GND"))
  (pad "39" thru_hole circle (at -0.1 0.17) (size 0.6 0.6) (drill 0.2) (layers "*.Cu" "F.Mask") (remove_unused_layers no) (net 2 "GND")
   (zone_connect 2))
  (pad "39" smd rect (at -0.1 0.87) (size 0.9 0.9) (layers "F.Cu" "F.Paste") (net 2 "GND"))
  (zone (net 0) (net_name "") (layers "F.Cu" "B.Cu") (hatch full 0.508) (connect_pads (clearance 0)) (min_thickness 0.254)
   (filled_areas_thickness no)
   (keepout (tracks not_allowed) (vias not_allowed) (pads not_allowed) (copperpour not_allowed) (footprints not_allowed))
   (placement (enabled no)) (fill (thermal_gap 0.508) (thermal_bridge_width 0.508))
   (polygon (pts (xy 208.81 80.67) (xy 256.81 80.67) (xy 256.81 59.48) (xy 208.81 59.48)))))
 (gr_rect (start 206.61 57.46) (end 258.75 104.39) (stroke (width 0.2) (type default)) (fill no) (layer "F.Cu"))
 (gr_rect (start 99.28 58.57) (end 153.71 106) (stroke (width 0.2) (type default)) (fill no) (layer "F.Cu"))
 (gr_rect (start 97.23 56.56) (end 155.12 107.53) (stroke (width 0.05) (type default)) (fill no) (layer "Edge.Cuts"))
 (segment (start 109.55 91.23) (end 117.8 91.23) (width 0.2) (layer "F.Cu") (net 1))
 (segment (start 117.8 91.23) (end 117.95 91.08) (width 0.2) (layer "F.Cu") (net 1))
 (segment (start 109.7 91.08) (end 109.55 91.23) (width 0.2) (layer "F.Cu") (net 1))
 (segment (start 215.74 91.35) (end 215.73 91.36) (width 0.2) (layer "F.Cu") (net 37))
 (segment (start 223.56 91.36) (end 224.06 90.86) (width 0.2) (layer "F.Cu") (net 37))
 (segment (start 215.73 91.36) (end 223.56 91.36) (width 0.2) (layer "F.Cu") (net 37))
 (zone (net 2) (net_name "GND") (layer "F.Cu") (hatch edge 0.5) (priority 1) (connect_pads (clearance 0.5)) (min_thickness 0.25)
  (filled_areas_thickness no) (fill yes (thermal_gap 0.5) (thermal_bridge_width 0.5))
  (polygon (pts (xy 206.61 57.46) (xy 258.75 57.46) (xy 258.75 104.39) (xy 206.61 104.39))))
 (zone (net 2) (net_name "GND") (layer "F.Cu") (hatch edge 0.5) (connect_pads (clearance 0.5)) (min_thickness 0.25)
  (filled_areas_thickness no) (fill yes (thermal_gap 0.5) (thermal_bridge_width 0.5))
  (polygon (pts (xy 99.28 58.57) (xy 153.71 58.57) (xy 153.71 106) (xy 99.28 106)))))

